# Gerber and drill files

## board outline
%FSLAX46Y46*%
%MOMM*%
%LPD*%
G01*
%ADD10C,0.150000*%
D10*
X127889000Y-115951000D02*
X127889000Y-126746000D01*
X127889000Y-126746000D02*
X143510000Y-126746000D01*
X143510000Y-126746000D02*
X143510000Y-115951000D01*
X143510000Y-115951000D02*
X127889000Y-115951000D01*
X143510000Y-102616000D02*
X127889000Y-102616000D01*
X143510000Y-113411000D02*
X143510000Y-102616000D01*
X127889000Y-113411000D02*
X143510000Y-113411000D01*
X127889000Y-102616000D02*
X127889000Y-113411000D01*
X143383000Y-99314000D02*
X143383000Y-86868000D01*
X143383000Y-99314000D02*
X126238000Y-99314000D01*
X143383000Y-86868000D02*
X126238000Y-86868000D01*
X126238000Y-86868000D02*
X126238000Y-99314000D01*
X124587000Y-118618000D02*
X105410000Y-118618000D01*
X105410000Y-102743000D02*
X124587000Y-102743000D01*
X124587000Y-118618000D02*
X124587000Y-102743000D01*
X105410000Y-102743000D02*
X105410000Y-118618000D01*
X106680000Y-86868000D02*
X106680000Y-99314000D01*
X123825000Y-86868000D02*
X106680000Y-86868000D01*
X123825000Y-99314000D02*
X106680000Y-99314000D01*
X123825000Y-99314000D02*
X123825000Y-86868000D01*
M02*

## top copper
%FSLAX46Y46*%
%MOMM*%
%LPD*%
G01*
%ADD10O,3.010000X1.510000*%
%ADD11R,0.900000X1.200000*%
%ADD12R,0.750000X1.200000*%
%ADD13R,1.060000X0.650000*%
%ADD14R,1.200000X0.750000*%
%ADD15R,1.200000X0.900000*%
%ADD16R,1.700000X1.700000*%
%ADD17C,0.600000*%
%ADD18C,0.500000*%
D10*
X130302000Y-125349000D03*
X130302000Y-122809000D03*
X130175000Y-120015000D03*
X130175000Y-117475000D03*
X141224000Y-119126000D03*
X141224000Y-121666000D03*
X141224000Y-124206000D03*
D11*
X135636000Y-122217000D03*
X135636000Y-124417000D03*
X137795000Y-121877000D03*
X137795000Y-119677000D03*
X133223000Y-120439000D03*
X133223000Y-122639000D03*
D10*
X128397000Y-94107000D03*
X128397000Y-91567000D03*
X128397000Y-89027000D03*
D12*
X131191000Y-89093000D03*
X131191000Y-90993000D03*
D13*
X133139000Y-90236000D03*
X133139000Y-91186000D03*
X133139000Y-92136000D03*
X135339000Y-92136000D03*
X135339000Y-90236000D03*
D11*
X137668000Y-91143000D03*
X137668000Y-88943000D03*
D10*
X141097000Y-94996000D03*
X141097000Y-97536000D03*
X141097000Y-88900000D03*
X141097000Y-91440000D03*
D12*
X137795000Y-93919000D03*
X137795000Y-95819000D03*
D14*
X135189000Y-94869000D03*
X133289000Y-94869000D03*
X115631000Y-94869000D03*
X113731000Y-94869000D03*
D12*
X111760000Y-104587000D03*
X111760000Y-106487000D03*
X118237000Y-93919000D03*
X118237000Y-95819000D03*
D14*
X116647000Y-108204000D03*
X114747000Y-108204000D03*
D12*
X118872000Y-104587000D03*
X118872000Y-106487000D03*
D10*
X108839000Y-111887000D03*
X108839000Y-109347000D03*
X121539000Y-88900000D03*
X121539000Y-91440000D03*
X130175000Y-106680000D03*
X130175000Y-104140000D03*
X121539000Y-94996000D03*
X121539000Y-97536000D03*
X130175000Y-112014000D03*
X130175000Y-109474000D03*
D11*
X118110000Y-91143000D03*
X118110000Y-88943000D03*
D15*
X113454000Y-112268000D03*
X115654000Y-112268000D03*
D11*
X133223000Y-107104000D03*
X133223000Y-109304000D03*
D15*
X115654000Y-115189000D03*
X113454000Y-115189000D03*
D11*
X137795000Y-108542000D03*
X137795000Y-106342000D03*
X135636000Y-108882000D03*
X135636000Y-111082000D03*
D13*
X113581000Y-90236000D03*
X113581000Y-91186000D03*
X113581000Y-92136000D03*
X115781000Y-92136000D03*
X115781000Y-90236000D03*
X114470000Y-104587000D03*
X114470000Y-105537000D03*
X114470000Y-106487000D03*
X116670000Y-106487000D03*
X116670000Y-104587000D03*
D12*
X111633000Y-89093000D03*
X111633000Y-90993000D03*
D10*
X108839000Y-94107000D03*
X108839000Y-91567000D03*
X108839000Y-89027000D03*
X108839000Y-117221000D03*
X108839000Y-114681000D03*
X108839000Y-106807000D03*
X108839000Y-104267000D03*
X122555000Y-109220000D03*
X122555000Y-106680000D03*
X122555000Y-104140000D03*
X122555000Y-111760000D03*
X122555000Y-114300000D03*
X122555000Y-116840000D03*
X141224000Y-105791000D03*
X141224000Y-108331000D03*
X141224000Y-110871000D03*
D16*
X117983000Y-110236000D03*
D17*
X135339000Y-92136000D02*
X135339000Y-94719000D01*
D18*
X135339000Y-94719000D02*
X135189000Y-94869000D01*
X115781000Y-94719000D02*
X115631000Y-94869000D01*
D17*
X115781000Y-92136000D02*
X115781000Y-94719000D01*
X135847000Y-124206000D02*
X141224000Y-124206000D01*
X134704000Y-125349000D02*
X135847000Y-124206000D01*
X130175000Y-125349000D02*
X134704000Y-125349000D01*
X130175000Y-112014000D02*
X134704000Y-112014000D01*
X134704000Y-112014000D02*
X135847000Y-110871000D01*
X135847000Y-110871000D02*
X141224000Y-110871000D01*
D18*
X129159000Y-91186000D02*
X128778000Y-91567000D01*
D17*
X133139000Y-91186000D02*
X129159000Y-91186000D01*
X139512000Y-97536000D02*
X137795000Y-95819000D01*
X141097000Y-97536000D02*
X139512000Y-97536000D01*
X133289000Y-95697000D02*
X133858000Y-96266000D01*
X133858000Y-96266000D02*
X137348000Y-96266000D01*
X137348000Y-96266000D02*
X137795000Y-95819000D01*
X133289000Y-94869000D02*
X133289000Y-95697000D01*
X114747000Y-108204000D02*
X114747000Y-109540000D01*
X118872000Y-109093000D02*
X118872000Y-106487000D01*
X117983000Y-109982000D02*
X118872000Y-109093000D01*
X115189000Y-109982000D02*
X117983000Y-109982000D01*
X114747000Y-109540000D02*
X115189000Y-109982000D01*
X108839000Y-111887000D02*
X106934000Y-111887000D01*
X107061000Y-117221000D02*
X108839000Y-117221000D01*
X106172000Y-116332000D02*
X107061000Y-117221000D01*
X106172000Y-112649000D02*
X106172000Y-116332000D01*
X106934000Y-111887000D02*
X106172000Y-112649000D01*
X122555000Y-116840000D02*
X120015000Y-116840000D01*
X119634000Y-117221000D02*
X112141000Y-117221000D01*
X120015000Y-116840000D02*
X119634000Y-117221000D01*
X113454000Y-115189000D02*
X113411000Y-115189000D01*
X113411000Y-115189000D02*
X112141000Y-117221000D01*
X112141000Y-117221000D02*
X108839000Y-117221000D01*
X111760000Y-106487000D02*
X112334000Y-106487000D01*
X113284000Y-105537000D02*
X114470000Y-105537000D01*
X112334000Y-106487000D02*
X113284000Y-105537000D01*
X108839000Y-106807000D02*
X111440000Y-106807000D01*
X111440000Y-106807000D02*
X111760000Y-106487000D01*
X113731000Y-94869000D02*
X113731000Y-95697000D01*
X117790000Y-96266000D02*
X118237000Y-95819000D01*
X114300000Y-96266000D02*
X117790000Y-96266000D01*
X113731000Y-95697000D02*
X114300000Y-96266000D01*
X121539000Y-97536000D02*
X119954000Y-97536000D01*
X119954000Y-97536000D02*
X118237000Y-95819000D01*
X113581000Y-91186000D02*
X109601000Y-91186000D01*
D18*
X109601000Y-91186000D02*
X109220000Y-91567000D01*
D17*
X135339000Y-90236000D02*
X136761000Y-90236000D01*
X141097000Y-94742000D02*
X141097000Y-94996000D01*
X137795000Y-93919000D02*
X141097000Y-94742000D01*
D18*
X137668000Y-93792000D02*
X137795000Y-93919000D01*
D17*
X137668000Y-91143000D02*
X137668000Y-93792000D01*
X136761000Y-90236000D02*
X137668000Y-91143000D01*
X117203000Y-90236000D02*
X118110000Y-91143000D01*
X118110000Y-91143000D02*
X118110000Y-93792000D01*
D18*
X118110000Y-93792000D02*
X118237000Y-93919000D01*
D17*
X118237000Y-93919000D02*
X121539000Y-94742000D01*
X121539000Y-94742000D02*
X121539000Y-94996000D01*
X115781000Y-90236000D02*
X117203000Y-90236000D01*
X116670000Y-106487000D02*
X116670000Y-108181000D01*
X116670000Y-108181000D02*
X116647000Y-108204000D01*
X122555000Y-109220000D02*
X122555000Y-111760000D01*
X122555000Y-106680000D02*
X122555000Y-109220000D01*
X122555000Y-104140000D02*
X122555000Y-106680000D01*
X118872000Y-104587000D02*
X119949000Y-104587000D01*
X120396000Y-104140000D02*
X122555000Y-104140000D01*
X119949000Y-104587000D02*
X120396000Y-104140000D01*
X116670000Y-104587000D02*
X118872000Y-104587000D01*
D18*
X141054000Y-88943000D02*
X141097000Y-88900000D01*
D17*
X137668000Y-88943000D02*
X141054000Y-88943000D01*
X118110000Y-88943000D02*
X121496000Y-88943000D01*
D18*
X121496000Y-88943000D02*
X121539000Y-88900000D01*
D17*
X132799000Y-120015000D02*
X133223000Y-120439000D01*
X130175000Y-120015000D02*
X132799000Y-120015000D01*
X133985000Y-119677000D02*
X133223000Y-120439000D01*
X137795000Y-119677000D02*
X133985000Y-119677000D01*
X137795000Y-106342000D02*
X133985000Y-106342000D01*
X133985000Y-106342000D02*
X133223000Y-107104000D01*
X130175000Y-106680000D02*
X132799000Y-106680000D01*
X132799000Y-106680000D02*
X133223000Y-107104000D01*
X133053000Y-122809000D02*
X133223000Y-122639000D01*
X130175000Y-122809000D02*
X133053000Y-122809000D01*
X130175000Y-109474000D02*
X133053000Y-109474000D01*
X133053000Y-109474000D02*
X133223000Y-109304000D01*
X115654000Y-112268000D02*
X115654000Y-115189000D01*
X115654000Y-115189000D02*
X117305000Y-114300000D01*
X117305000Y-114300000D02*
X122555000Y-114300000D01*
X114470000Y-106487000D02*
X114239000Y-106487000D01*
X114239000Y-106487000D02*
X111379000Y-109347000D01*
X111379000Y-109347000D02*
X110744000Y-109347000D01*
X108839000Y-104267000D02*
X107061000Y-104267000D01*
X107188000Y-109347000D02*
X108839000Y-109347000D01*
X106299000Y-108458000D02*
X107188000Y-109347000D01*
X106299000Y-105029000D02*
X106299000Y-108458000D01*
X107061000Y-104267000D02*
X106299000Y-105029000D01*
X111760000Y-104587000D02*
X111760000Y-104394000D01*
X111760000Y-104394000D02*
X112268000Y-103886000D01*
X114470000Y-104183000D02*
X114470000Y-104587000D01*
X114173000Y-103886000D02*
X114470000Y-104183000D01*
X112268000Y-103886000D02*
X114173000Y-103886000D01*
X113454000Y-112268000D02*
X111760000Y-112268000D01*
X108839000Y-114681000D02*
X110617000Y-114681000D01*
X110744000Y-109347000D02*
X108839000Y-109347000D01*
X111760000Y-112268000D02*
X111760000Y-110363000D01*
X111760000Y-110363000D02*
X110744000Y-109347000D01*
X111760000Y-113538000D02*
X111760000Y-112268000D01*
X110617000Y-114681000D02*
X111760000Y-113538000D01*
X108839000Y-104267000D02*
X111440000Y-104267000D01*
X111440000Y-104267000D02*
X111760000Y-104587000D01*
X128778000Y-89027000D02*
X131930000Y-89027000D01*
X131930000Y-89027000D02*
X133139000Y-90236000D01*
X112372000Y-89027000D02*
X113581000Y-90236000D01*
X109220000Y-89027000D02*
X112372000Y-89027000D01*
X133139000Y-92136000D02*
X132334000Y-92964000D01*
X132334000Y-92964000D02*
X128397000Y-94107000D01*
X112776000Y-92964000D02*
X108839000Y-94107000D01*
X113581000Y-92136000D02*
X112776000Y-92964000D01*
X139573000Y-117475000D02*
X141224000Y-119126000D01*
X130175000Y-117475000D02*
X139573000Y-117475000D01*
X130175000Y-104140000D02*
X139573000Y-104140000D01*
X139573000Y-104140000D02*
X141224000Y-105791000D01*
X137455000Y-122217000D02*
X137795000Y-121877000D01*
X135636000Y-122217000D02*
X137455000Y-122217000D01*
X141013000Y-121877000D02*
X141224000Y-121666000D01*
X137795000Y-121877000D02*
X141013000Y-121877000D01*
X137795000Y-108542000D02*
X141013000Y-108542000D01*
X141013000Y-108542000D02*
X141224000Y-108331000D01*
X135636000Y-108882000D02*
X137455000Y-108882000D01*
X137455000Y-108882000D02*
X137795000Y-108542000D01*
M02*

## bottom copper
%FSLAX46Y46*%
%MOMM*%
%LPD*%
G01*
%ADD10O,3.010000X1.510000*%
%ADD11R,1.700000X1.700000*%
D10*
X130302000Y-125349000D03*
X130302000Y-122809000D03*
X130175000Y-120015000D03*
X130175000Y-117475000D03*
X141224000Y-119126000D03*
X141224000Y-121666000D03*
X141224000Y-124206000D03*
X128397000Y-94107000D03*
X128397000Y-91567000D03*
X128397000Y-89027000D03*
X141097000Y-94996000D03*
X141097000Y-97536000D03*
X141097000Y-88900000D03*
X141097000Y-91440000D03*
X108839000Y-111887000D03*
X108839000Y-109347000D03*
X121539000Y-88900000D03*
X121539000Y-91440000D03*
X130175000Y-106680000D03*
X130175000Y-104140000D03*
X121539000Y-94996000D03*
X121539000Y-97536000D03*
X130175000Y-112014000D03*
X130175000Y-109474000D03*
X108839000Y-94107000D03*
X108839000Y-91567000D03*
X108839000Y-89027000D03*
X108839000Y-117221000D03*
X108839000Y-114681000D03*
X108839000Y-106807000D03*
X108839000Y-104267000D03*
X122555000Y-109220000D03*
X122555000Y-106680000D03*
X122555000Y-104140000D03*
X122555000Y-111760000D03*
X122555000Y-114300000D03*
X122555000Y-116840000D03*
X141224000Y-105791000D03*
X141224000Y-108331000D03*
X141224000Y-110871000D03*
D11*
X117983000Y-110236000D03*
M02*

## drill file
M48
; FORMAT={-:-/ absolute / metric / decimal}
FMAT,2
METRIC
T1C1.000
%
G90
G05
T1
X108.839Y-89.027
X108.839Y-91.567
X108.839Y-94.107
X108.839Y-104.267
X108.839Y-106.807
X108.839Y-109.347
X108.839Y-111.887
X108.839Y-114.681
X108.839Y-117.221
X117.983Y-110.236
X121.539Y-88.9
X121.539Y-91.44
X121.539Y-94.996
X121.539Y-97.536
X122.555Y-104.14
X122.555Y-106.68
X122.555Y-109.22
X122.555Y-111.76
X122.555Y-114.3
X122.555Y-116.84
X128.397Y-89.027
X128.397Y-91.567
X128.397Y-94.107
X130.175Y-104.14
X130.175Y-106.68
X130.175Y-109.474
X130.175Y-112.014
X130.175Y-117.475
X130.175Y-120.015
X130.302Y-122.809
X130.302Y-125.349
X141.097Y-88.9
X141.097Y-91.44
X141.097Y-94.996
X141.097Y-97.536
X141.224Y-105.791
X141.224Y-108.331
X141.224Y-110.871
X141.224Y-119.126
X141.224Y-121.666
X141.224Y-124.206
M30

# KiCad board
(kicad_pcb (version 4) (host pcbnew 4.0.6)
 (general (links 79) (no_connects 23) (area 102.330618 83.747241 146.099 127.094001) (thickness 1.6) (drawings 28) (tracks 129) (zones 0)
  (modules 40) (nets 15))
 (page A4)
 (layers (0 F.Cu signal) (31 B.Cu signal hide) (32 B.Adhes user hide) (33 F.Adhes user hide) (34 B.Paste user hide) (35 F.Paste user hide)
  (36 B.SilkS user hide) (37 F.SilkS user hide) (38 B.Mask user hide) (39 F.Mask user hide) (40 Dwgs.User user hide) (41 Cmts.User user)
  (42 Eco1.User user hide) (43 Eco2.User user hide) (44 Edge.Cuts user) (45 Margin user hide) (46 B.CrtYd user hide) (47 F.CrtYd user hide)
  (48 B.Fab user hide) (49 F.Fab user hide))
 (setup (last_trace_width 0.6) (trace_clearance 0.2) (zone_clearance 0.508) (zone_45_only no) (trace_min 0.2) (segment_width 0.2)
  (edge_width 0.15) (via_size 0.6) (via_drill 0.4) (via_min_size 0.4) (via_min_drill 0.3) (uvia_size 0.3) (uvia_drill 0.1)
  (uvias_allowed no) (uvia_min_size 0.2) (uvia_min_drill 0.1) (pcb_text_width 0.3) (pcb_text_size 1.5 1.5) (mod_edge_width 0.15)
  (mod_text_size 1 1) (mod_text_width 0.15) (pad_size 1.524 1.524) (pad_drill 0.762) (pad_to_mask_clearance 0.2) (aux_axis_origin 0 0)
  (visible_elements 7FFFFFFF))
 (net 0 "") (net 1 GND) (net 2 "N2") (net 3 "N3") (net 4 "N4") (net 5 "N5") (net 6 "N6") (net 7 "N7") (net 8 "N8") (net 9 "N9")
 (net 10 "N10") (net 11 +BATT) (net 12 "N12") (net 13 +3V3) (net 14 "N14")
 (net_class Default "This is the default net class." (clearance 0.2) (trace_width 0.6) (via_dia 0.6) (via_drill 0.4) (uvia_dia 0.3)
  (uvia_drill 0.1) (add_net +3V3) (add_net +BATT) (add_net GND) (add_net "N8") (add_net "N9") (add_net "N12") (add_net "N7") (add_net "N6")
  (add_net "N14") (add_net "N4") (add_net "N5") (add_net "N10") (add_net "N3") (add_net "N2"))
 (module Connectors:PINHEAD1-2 (layer F.Cu) (at 130.302 125.349 90)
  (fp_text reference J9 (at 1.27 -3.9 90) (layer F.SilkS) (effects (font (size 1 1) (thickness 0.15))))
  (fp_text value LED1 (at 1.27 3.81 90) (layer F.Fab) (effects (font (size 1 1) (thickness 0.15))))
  (pad 1 thru_hole oval (at 0 0 90) (size 1.51 3.01) (drill 1) (layers *.Cu *.Mask) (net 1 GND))
  (pad 2 thru_hole oval (at 2.54 0 90) (size 1.51 3.01) (drill 1) (layers *.Cu *.Mask) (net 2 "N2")))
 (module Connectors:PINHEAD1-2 (layer F.Cu) (at 130.175 120.015 90)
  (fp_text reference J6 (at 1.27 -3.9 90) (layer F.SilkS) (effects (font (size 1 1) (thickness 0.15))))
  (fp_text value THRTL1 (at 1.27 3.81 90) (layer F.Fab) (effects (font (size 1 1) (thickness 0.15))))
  (pad 1 thru_hole oval (at 0 0 90) (size 1.51 3.01) (drill 1) (layers *.Cu *.Mask) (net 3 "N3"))
  (pad 2 thru_hole oval (at 2.54 0 90) (size 1.51 3.01) (drill 1) (layers *.Cu *.Mask) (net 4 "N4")))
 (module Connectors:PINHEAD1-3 (layer F.Cu) (at 141.224 119.126 270)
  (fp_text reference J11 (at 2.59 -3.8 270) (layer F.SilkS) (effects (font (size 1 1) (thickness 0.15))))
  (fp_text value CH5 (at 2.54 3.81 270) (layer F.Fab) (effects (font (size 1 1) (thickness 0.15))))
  (pad 1 thru_hole oval (at 0 0 270) (size 1.51 3.01) (drill 1) (layers *.Cu *.Mask) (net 4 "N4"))
  (pad 2 thru_hole oval (at 2.54 0 270) (size 1.51 3.01) (drill 1) (layers *.Cu *.Mask) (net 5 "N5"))
  (pad 3 thru_hole oval (at 5.08 0 270) (size 1.51 3.01) (drill 1) (layers *.Cu *.Mask) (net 1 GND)))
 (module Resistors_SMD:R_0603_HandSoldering (layer F.Cu) (at 135.636 123.317 270)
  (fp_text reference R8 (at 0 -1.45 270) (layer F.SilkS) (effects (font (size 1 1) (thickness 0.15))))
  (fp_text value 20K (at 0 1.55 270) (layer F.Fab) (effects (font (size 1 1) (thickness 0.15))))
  (pad 1 smd rect (at -1.1 0 270) (size 1.2 0.9) (layers F.Cu F.Paste F.Mask) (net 5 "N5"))
  (pad 2 smd rect (at 1.1 0 270) (size 1.2 0.9) (layers F.Cu F.Paste F.Mask) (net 1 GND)))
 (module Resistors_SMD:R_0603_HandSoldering (layer F.Cu) (at 137.795 120.777 90)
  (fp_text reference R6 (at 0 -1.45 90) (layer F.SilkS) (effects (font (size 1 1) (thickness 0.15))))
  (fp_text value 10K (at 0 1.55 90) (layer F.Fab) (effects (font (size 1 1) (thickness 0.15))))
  (pad 1 smd rect (at -1.1 0 90) (size 1.2 0.9) (layers F.Cu F.Paste F.Mask) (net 5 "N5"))
  (pad 2 smd rect (at 1.1 0 90) (size 1.2 0.9) (layers F.Cu F.Paste F.Mask) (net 3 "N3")))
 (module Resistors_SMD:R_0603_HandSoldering (layer F.Cu) (at 133.223 121.539 270)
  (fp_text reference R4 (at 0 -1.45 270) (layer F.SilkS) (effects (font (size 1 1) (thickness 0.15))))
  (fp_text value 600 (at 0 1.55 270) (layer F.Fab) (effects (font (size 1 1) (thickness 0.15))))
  (pad 1 smd rect (at -1.1 0 270) (size 1.2 0.9) (layers F.Cu F.Paste F.Mask) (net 3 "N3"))
  (pad 2 smd rect (at 1.1 0 270) (size 1.2 0.9) (layers F.Cu F.Paste F.Mask) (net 2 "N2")))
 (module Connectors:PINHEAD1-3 (layer F.Cu) (at 128.397 94.107 90)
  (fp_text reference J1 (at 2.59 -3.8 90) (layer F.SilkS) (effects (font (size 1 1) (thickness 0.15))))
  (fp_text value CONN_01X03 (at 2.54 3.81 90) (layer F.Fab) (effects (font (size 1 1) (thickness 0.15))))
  (pad 1 thru_hole oval (at 0 0 90) (size 1.51 3.01) (drill 1) (layers *.Cu *.Mask) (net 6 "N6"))
  (pad 2 thru_hole oval (at 2.54 0 90) (size 1.51 3.01) (drill 1) (layers *.Cu *.Mask) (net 1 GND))
  (pad 3 thru_hole oval (at 5.08 0 90) (size 1.51 3.01) (drill 1) (layers *.Cu *.Mask) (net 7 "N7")))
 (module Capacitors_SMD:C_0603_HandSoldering (layer F.Cu) (at 131.191 90.043 270)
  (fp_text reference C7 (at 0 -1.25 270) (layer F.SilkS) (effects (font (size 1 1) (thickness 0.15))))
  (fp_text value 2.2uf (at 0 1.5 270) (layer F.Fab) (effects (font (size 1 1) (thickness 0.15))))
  (pad 1 smd rect (at -0.95 0 270) (size 1.2 0.75) (layers F.Cu F.Paste F.Mask) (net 7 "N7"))
  (pad 2 smd rect (at 0.95 0 270) (size 1.2 0.75) (layers F.Cu F.Paste F.Mask) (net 1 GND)))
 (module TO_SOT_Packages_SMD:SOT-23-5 (layer F.Cu) (at 134.239 91.186)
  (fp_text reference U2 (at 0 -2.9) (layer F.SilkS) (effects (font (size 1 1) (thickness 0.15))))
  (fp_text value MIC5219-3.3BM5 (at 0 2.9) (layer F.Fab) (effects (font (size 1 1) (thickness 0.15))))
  (pad 1 smd rect (at -1.1 -0.95) (size 1.06 0.65) (layers F.Cu F.Paste F.Mask) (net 7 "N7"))
  (pad 2 smd rect (at -1.1 0) (size 1.06 0.65) (layers F.Cu F.Paste F.Mask) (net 1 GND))
  (pad 3 smd rect (at -1.1 0.95) (size 1.06 0.65) (layers F.Cu F.Paste F.Mask) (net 6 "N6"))
  (pad 4 smd rect (at 1.1 0.95) (size 1.06 0.65) (layers F.Cu F.Paste F.Mask) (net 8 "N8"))
  (pad 5 smd rect (at 1.1 -0.95) (size 1.06 0.65) (layers F.Cu F.Paste F.Mask) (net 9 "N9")))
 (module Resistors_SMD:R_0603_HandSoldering (layer F.Cu) (at 137.668 90.043 90)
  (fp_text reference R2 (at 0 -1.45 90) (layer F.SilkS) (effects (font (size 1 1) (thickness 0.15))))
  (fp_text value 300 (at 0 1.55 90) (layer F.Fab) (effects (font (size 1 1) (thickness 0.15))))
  (pad 1 smd rect (at -1.1 0 90) (size 1.2 0.9) (layers F.Cu F.Paste F.Mask) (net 9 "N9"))
  (pad 2 smd rect (at 1.1 0 90) (size 1.2 0.9) (layers F.Cu F.Paste F.Mask) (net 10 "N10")))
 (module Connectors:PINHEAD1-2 (layer F.Cu) (at 141.097 94.996 270)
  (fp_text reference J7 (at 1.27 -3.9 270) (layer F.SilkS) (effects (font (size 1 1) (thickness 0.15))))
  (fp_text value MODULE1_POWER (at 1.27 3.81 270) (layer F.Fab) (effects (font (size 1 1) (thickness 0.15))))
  (pad 1 thru_hole oval (at 0 0 270) (size 1.51 3.01) (drill 1) (layers *.Cu *.Mask) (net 9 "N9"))
  (pad 2 thru_hole oval (at 2.54 0 270) (size 1.51 3.01) (drill 1) (layers *.Cu *.Mask) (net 1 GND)))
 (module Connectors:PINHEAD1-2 (layer F.Cu) (at 141.097 88.9 270)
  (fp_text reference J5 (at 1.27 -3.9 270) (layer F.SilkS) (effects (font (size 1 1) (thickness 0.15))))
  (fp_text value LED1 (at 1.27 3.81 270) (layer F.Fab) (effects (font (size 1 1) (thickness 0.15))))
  (pad 1 thru_hole oval (at 0 0 270) (size 1.51 3.01) (drill 1) (layers *.Cu *.Mask) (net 10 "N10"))
  (pad 2 thru_hole oval (at 2.54 0 270) (size 1.51 3.01) (drill 1) (layers *.Cu *.Mask) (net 1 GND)))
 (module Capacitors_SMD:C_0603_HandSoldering (layer F.Cu) (at 137.795 94.869 270)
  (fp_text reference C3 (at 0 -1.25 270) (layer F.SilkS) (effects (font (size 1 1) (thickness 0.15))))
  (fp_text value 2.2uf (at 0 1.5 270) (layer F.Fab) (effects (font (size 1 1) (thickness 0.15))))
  (pad 1 smd rect (at -0.95 0 270) (size 1.2 0.75) (layers F.Cu F.Paste F.Mask) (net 9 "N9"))
  (pad 2 smd rect (at 0.95 0 270) (size 1.2 0.75) (layers F.Cu F.Paste F.Mask) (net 1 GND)))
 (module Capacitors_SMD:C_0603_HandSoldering (layer F.Cu) (at 134.239 94.869 180)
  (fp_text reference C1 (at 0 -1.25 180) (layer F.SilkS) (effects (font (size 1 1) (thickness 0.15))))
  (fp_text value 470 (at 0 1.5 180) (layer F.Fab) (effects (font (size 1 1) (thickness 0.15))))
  (pad 1 smd rect (at -0.95 0 180) (size 1.2 0.75) (layers F.Cu F.Paste F.Mask) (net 8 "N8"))
  (pad 2 smd rect (at 0.95 0 180) (size 1.2 0.75) (layers F.Cu F.Paste F.Mask) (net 1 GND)))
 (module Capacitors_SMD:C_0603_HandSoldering (layer F.Cu) (at 114.681 94.869 180)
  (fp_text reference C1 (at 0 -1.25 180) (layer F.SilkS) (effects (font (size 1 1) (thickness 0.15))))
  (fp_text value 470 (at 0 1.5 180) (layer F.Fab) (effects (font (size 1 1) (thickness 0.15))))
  (pad 1 smd rect (at -0.95 0 180) (size 1.2 0.75) (layers F.Cu F.Paste F.Mask) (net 8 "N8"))
  (pad 2 smd rect (at 0.95 0 180) (size 1.2 0.75) (layers F.Cu F.Paste F.Mask) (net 1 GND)))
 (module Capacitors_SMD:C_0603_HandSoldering (layer F.Cu) (at 111.76 105.537 270)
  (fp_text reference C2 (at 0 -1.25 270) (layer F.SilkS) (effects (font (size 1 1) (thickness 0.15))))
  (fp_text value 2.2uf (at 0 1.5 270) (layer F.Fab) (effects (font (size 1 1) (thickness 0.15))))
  (pad 1 smd rect (at -0.95 0 270) (size 1.2 0.75) (layers F.Cu F.Paste F.Mask) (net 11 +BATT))
  (pad 2 smd rect (at 0.95 0 270) (size 1.2 0.75) (layers F.Cu F.Paste F.Mask) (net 1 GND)))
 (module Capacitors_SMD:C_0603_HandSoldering (layer F.Cu) (at 118.237 94.869 270)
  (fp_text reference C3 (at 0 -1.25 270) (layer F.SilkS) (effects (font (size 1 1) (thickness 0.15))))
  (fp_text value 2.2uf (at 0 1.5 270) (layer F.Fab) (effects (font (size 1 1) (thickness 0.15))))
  (pad 1 smd rect (at -0.95 0 270) (size 1.2 0.75) (layers F.Cu F.Paste F.Mask) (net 9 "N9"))
  (pad 2 smd rect (at 0.95 0 270) (size 1.2 0.75) (layers F.Cu F.Paste F.Mask) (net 1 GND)))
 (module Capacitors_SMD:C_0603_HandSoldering (layer F.Cu) (at 115.697 108.204 180)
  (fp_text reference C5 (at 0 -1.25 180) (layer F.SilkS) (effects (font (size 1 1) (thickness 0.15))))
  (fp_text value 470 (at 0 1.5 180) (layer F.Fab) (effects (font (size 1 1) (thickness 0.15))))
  (pad 1 smd rect (at -0.95 0 180) (size 1.2 0.75) (layers F.Cu F.Paste F.Mask) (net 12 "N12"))
  (pad 2 smd rect (at 0.95 0 180) (size 1.2 0.75) (layers F.Cu F.Paste F.Mask) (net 1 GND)))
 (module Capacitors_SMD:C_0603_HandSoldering (layer F.Cu) (at 118.872 105.537 270)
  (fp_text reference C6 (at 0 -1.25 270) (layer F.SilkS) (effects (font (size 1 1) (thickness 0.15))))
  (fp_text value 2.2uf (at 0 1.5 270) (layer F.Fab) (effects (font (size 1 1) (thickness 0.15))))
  (pad 1 smd rect (at -0.95 0 270) (size 1.2 0.75) (layers F.Cu F.Paste F.Mask) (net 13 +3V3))
  (pad 2 smd rect (at 0.95 0 270) (size 1.2 0.75) (layers F.Cu F.Paste F.Mask) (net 1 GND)))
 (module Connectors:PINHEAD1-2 (layer F.Cu) (at 108.839 111.887 90)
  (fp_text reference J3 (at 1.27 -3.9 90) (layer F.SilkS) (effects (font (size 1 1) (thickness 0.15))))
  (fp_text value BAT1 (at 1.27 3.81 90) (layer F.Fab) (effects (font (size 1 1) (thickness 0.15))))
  (pad 1 thru_hole oval (at 0 0 90) (size 1.51 3.01) (drill 1) (layers *.Cu *.Mask) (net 1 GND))
  (pad 2 thru_hole oval (at 2.54 0 90) (size 1.51 3.01) (drill 1) (layers *.Cu *.Mask) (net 11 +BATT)))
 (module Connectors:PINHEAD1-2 (layer F.Cu) (at 121.539 88.9 270)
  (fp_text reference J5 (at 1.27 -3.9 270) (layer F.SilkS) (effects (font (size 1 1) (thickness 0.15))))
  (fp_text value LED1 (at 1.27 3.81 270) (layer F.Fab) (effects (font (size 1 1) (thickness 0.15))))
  (pad 1 thru_hole oval (at 0 0 270) (size 1.51 3.01) (drill 1) (layers *.Cu *.Mask) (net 10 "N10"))
  (pad 2 thru_hole oval (at 2.54 0 270) (size 1.51 3.01) (drill 1) (layers *.Cu *.Mask) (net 1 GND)))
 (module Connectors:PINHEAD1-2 (layer F.Cu) (at 130.175 106.68 90)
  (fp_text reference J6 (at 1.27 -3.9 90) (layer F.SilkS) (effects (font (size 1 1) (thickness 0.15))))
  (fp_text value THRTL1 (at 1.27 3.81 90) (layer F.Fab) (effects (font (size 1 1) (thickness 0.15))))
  (pad 1 thru_hole oval (at 0 0 90) (size 1.51 3.01) (drill 1) (layers *.Cu *.Mask) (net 3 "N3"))
  (pad 2 thru_hole oval (at 2.54 0 90) (size 1.51 3.01) (drill 1) (layers *.Cu *.Mask) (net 4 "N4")))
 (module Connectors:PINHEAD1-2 (layer F.Cu) (at 121.539 94.996 270)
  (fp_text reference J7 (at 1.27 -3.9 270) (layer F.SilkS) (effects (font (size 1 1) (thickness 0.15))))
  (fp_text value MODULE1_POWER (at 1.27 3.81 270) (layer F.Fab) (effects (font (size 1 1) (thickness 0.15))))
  (pad 1 thru_hole oval (at 0 0 270) (size 1.51 3.01) (drill 1) (layers *.Cu *.Mask) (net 9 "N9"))
  (pad 2 thru_hole oval (at 2.54 0 270) (size 1.51 3.01) (drill 1) (layers *.Cu *.Mask) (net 1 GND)))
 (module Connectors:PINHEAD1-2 (layer F.Cu) (at 130.175 112.014 90)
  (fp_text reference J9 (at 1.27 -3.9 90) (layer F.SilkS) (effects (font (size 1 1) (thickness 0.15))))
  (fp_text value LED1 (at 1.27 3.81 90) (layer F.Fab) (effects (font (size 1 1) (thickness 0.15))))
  (pad 1 thru_hole oval (at 0 0 90) (size 1.51 3.01) (drill 1) (layers *.Cu *.Mask) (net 1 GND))
  (pad 2 thru_hole oval (at 2.54 0 90) (size 1.51 3.01) (drill 1) (layers *.Cu *.Mask) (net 2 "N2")))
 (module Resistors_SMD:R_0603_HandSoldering (layer F.Cu) (at 118.11 90.043 90)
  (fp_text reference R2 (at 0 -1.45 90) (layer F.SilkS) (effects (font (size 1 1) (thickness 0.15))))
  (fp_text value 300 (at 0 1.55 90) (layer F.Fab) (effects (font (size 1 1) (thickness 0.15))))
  (pad 1 smd rect (at -1.1 0 90) (size 1.2 0.9) (layers F.Cu F.Paste F.Mask) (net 9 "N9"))
  (pad 2 smd rect (at 1.1 0 90) (size 1.2 0.9) (layers F.Cu F.Paste F.Mask) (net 10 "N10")))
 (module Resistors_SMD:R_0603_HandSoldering (layer F.Cu) (at 114.554 112.268)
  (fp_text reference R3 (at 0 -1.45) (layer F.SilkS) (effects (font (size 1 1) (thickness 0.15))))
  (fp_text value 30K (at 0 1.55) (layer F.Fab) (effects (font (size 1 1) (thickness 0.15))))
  (pad 1 smd rect (at -1.1 0) (size 1.2 0.9) (layers F.Cu F.Paste F.Mask) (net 11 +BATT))
  (pad 2 smd rect (at 1.1 0) (size 1.2 0.9) (layers F.Cu F.Paste F.Mask) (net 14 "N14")))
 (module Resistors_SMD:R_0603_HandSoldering (layer F.Cu) (at 133.223 108.204 270)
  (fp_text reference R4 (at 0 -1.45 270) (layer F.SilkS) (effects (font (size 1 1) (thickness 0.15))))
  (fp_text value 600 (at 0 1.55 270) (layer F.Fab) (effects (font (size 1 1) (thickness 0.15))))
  (pad 1 smd rect (at -1.1 0 270) (size 1.2 0.9) (layers F.Cu F.Paste F.Mask) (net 3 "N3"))
  (pad 2 smd rect (at 1.1 0 270) (size 1.2 0.9) (layers F.Cu F.Paste F.Mask) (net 2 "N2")))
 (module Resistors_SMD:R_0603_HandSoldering (layer F.Cu) (at 114.554 115.189 180)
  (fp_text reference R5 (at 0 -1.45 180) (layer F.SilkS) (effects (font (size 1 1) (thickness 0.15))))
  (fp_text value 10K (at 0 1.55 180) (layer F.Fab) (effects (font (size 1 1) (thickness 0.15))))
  (pad 1 smd rect (at -1.1 0 180) (size 1.2 0.9) (layers F.Cu F.Paste F.Mask) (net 14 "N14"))
  (pad 2 smd rect (at 1.1 0 180) (size 1.2 0.9) (layers F.Cu F.Paste F.Mask) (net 1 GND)))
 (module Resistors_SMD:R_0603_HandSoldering (layer F.Cu) (at 137.795 107.442 90)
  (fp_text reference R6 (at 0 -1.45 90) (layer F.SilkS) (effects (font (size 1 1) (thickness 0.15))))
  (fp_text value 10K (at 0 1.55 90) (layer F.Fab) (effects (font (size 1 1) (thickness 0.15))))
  (pad 1 smd rect (at -1.1 0 90) (size 1.2 0.9) (layers F.Cu F.Paste F.Mask) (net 5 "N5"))
  (pad 2 smd rect (at 1.1 0 90) (size 1.2 0.9) (layers F.Cu F.Paste F.Mask) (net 3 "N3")))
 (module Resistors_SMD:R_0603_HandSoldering (layer F.Cu) (at 135.636 109.982 270)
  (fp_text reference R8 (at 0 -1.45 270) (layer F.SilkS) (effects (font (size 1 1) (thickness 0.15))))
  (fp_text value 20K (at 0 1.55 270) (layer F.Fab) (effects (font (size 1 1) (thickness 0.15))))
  (pad 1 smd rect (at -1.1 0 270) (size 1.2 0.9) (layers F.Cu F.Paste F.Mask) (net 5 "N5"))
  (pad 2 smd rect (at 1.1 0 270) (size 1.2 0.9) (layers F.Cu F.Paste F.Mask) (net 1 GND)))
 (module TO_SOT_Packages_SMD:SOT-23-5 (layer F.Cu) (at 114.681 91.186)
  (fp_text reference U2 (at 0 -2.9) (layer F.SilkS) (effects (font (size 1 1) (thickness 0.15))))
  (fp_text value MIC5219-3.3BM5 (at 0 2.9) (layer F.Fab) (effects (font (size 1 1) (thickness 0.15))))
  (pad 1 smd rect (at -1.1 -0.95) (size 1.06 0.65) (layers F.Cu F.Paste F.Mask) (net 7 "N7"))
  (pad 2 smd rect (at -1.1 0) (size 1.06 0.65) (layers F.Cu F.Paste F.Mask) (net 1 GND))
  (pad 3 smd rect (at -1.1 0.95) (size 1.06 0.65) (layers F.Cu F.Paste F.Mask) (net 6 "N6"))
  (pad 4 smd rect (at 1.1 0.95) (size 1.06 0.65) (layers F.Cu F.Paste F.Mask) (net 8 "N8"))
  (pad 5 smd rect (at 1.1 -0.95) (size 1.06 0.65) (layers F.Cu F.Paste F.Mask) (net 9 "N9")))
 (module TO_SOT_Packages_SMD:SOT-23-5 (layer F.Cu) (at 115.57 105.537)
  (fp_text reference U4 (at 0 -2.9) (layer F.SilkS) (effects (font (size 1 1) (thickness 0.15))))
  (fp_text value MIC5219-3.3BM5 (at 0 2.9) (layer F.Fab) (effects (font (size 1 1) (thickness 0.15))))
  (pad 1 smd rect (at -1.1 -0.95) (size 1.06 0.65) (layers F.Cu F.Paste F.Mask) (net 11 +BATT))
  (pad 2 smd rect (at -1.1 0) (size 1.06 0.65) (layers F.Cu F.Paste F.Mask) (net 1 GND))
  (pad 3 smd rect (at -1.1 0.95) (size 1.06 0.65) (layers F.Cu F.Paste F.Mask) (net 11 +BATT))
  (pad 4 smd rect (at 1.1 0.95) (size 1.06 0.65) (layers F.Cu F.Paste F.Mask) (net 12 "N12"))
  (pad 5 smd rect (at 1.1 -0.95) (size 1.06 0.65) (layers F.Cu F.Paste F.Mask) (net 13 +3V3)))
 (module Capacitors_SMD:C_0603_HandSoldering (layer F.Cu) (at 111.633 90.043 270)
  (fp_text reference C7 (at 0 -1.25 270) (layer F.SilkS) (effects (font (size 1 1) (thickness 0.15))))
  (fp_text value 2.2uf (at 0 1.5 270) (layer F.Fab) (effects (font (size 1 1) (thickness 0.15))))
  (pad 1 smd rect (at -0.95 0 270) (size 1.2 0.75) (layers F.Cu F.Paste F.Mask) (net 7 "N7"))
  (pad 2 smd rect (at 0.95 0 270) (size 1.2 0.75) (layers F.Cu F.Paste F.Mask) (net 1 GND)))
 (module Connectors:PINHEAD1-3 (layer F.Cu) (at 108.839 94.107 90)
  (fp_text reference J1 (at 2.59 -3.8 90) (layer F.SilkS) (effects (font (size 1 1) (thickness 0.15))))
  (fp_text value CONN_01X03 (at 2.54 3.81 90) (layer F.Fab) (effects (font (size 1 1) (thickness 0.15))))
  (pad 1 thru_hole oval (at 0 0 90) (size 1.51 3.01) (drill 1) (layers *.Cu *.Mask) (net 6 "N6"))
  (pad 2 thru_hole oval (at 2.54 0 90) (size 1.51 3.01) (drill 1) (layers *.Cu *.Mask) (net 1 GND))
  (pad 3 thru_hole oval (at 5.08 0 90) (size 1.51 3.01) (drill 1) (layers *.Cu *.Mask) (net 7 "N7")))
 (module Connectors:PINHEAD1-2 (layer F.Cu) (at 108.839 117.221 90)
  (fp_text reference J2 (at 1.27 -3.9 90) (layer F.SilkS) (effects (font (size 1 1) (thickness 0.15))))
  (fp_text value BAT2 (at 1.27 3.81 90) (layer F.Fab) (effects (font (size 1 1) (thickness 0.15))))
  (pad 1 thru_hole oval (at 0 0 90) (size 1.51 3.01) (drill 1) (layers *.Cu *.Mask) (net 1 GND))
  (pad 2 thru_hole oval (at 2.54 0 90) (size 1.51 3.01) (drill 1) (layers *.Cu *.Mask) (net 11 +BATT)))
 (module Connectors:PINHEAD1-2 (layer F.Cu) (at 108.839 106.807 90)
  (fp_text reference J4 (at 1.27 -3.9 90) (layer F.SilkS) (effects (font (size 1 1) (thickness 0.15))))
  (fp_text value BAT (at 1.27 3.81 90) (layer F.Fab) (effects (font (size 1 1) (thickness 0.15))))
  (pad 1 thru_hole oval (at 0 0 90) (size 1.51 3.01) (drill 1) (layers *.Cu *.Mask) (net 1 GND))
  (pad 2 thru_hole oval (at 2.54 0 90) (size 1.51 3.01) (drill 1) (layers *.Cu *.Mask) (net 11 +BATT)))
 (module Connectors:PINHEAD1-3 (layer F.Cu) (at 122.555 109.22 90)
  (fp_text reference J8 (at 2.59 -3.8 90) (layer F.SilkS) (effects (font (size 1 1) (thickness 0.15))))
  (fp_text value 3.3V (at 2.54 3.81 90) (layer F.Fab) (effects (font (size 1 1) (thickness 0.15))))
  (pad 1 thru_hole oval (at 0 0 90) (size 1.51 3.01) (drill 1) (layers *.Cu *.Mask) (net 13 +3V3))
  (pad 2 thru_hole oval (at 2.54 0 90) (size 1.51 3.01) (drill 1) (layers *.Cu *.Mask) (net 13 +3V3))
  (pad 3 thru_hole oval (at 5.08 0 90) (size 1.51 3.01) (drill 1) (layers *.Cu *.Mask) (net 13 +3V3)))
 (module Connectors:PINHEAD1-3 (layer F.Cu) (at 122.555 111.76 270)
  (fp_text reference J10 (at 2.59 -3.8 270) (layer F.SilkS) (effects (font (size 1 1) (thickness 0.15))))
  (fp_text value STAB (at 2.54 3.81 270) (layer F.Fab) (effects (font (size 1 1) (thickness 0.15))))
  (pad 1 thru_hole oval (at 0 0 270) (size 1.51 3.01) (drill 1) (layers *.Cu *.Mask) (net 13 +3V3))
  (pad 2 thru_hole oval (at 2.54 0 270) (size 1.51 3.01) (drill 1) (layers *.Cu *.Mask) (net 14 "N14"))
  (pad 3 thru_hole oval (at 5.08 0 270) (size 1.51 3.01) (drill 1) (layers *.Cu *.Mask) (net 1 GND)))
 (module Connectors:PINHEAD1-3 (layer F.Cu) (at 141.224 105.791 270)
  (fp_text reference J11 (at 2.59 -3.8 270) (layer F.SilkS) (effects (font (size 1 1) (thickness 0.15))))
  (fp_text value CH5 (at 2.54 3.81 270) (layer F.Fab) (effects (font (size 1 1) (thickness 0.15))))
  (pad 1 thru_hole oval (at 0 0 270) (size 1.51 3.01) (drill 1) (layers *.Cu *.Mask) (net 4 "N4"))
  (pad 2 thru_hole oval (at 2.54 0 270) (size 1.51 3.01) (drill 1) (layers *.Cu *.Mask) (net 5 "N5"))
  (pad 3 thru_hole oval (at 5.08 0 270) (size 1.51 3.01) (drill 1) (layers *.Cu *.Mask) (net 1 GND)))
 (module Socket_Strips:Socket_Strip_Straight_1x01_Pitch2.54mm (layer F.Cu) (at 117.983 110.236)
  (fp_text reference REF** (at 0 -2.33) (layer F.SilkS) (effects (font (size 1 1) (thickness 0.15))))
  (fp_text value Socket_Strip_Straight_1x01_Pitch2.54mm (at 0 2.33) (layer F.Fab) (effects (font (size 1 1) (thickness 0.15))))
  (pad 1 thru_hole rect (at 0 0) (size 1.7 1.7) (drill 1) (layers *.Cu *.Mask)))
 (gr_line (start 127.889 115.951) (end 127.889 126.746) (angle 90) (layer Edge.Cuts) (width 0.15))
 (gr_line (start 127.889 126.746) (end 143.51 126.746) (angle 90) (layer Edge.Cuts) (width 0.15))
 (gr_line (start 143.51 126.746) (end 143.51 115.951) (angle 90) (layer Edge.Cuts) (width 0.15))
 (gr_line (start 143.51 115.951) (end 127.889 115.951) (angle 90) (layer Edge.Cuts) (width 0.15))
 (gr_line (start 143.51 102.616) (end 127.889 102.616) (angle 90) (layer Edge.Cuts) (width 0.15))
 (gr_line (start 143.51 113.411) (end 143.51 102.616) (angle 90) (layer Edge.Cuts) (width 0.15))
 (gr_line (start 127.889 113.411) (end 143.51 113.411) (angle 90) (layer Edge.Cuts) (width 0.15))
 (gr_line (start 127.889 102.616) (end 127.889 113.411) (angle 90) (layer Edge.Cuts) (width 0.15))
 (gr_line (start 143.383 99.314) (end 143.383 86.868) (angle 90) (layer Edge.Cuts) (width 0.15))
 (gr_line (start 143.383 99.314) (end 126.238 99.314) (angle 90) (layer Edge.Cuts) (width 0.15))
 (gr_line (start 143.383 86.868) (end 126.238 86.868) (angle 90) (layer Edge.Cuts) (width 0.15))
 (gr_line (start 126.238 86.868) (end 126.238 99.314) (angle 90) (layer Edge.Cuts) (width 0.15))
 (gr_line (start 124.587 118.618) (end 105.41 118.618) (angle 90) (layer Edge.Cuts) (width 0.15))
 (gr_line (start 105.41 102.743) (end 124.587 102.743) (angle 90) (layer Edge.Cuts) (width 0.15))
 (gr_line (start 124.587 118.618) (end 124.587 102.743) (angle 90) (layer Edge.Cuts) (width 0.15))
 (gr_line (start 105.41 102.743) (end 105.41 118.618) (angle 90) (layer Edge.Cuts) (width 0.15))
 (gr_line (start 106.68 86.868) (end 106.68 99.314) (angle 90) (layer Edge.Cuts) (width 0.15))
 (gr_line (start 123.825 86.868) (end 106.68 86.868) (angle 90) (layer Edge.Cuts) (width 0.15))
 (gr_line (start 123.825 99.314) (end 106.68 99.314) (angle 90) (layer Edge.Cuts) (width 0.15))
 (gr_line (start 123.825 99.314) (end 123.825 86.868) (angle 90) (layer Edge.Cuts) (width 0.15))
 (segment (start 135.339 92.136) (end 135.339 94.719) (width 0.6) (layer F.Cu) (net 8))
 (segment (start 135.339 94.719) (end 135.189 94.869) (width 0.5) (layer F.Cu) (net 8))
 (segment (start 115.781 94.719) (end 115.631 94.869) (width 0.5) (layer F.Cu) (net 8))
 (segment (start 115.781 92.136) (end 115.781 94.719) (width 0.6) (layer F.Cu) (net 8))
 (segment (start 135.847 124.206) (end 141.224 124.206) (width 0.6) (layer F.Cu) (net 1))
 (segment (start 134.704 125.349) (end 135.847 124.206) (width 0.6) (layer F.Cu) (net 1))
 (segment (start 130.175 125.349) (end 134.704 125.349) (width 0.6) (layer F.Cu) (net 1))
 (segment (start 130.175 112.014) (end 134.704 112.014) (width 0.6) (layer F.Cu) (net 1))
 (segment (start 134.704 112.014) (end 135.847 110.871) (width 0.6) (layer F.Cu) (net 1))
 (segment (start 135.847 110.871) (end 141.224 110.871) (width 0.6) (layer F.Cu) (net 1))
 (segment (start 129.159 91.186) (end 128.778 91.567) (width 0.5) (layer F.Cu) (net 1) (status 30))
 (segment (start 133.139 91.186) (end 129.159 91.186) (width 0.6) (layer F.Cu) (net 1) (status 20))
 (segment (start 139.512 97.536) (end 137.795 95.819) (width 0.6) (layer F.Cu) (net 1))
 (segment (start 141.097 97.536) (end 139.512 97.536) (width 0.6) (layer F.Cu) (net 1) (status 10))
 (segment (start 133.289 95.697) (end 133.858 96.266) (width 0.6) (layer F.Cu) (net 1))
 (segment (start 133.858 96.266) (end 137.348 96.266) (width 0.6) (layer F.Cu) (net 1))
 (segment (start 137.348 96.266) (end 137.795 95.819) (width 0.6) (layer F.Cu) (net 1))
 (segment (start 133.289 94.869) (end 133.289 95.697) (width 0.6) (layer F.Cu) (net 1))
 (segment (start 114.747 108.204) (end 114.747 109.54) (width 0.6) (layer F.Cu) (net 1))
 (segment (start 118.872 109.093) (end 118.872 106.487) (width 0.6) (layer F.Cu) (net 1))
 (segment (start 117.983 109.982) (end 118.872 109.093) (width 0.6) (layer F.Cu) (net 1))
 (segment (start 115.189 109.982) (end 117.983 109.982) (width 0.6) (layer F.Cu) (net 1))
 (segment (start 114.747 109.54) (end 115.189 109.982) (width 0.6) (layer F.Cu) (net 1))
 (segment (start 108.839 111.887) (end 106.934 111.887) (width 0.6) (layer F.Cu) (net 1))
 (segment (start 107.061 117.221) (end 108.839 117.221) (width 0.6) (layer F.Cu) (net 1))
 (segment (start 106.172 116.332) (end 107.061 117.221) (width 0.6) (layer F.Cu) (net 1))
 (segment (start 106.172 112.649) (end 106.172 116.332) (width 0.6) (layer F.Cu) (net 1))
 (segment (start 106.934 111.887) (end 106.172 112.649) (width 0.6) (layer F.Cu) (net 1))
 (segment (start 122.555 116.84) (end 120.015 116.84) (width 0.6) (layer F.Cu) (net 1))
 (segment (start 119.634 117.221) (end 112.141 117.221) (width 0.6) (layer F.Cu) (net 1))
 (segment (start 120.015 116.84) (end 119.634 117.221) (width 0.6) (layer F.Cu) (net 1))
 (segment (start 113.454 115.189) (end 113.411 115.189) (width 0.6) (layer F.Cu) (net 1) (status 30))
 (segment (start 113.411 115.189) (end 112.141 117.221) (width 0.6) (layer F.Cu) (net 1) (status 10))
 (segment (start 112.141 117.221) (end 108.839 117.221) (width 0.6) (layer F.Cu) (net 1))
 (segment (start 111.76 106.487) (end 112.334 106.487) (width 0.6) (layer F.Cu) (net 1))
 (segment (start 113.284 105.537) (end 114.47 105.537) (width 0.6) (layer F.Cu) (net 1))
 (segment (start 112.334 106.487) (end 113.284 105.537) (width 0.6) (layer F.Cu) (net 1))
 (segment (start 108.839 106.807) (end 111.44 106.807) (width 0.6) (layer F.Cu) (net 1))
 (segment (start 111.44 106.807) (end 111.76 106.487) (width 0.6) (layer F.Cu) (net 1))
 (segment (start 113.731 94.869) (end 113.731 95.697) (width 0.6) (layer F.Cu) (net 1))
 (segment (start 117.79 96.266) (end 118.237 95.819) (width 0.6) (layer F.Cu) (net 1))
 (segment (start 114.3 96.266) (end 117.79 96.266) (width 0.6) (layer F.Cu) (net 1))
 (segment (start 113.731 95.697) (end 114.3 96.266) (width 0.6) (layer F.Cu) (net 1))
 (segment (start 121.539 97.536) (end 119.954 97.536) (width 0.6) (layer F.Cu) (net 1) (status 10))
 (segment (start 119.954 97.536) (end 118.237 95.819) (width 0.6) (layer F.Cu) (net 1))
 (segment (start 113.581 91.186) (end 109.601 91.186) (width 0.6) (layer F.Cu) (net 1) (status 20))
 (segment (start 109.601 91.186) (end 109.22 91.567) (width 0.5) (layer F.Cu) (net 1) (status 30))
 (segment (start 135.339 90.236) (end 136.761 90.236) (width 0.6) (layer F.Cu) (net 9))
 (segment (start 141.097 94.742) (end 141.097 94.996) (width 0.6) (layer F.Cu) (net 9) (status 20))
 (segment (start 137.795 93.919) (end 141.097 94.742) (width 0.6) (layer F.Cu) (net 9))
 (segment (start 137.668 93.792) (end 137.795 93.919) (width 0.5) (layer F.Cu) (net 9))
 (segment (start 137.668 91.143) (end 137.668 93.792) (width 0.6) (layer F.Cu) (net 9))
 (segment (start 136.761 90.236) (end 137.668 91.143) (width 0.6) (layer F.Cu) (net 9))
 (segment (start 117.203 90.236) (end 118.11 91.143) (width 0.6) (layer F.Cu) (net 9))
 (segment (start 118.11 91.143) (end 118.11 93.792) (width 0.6) (layer F.Cu) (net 9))
 (segment (start 118.11 93.792) (end 118.237 93.919) (width 0.5) (layer F.Cu) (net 9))
 (segment (start 118.237 93.919) (end 121.539 94.742) (width 0.6) (layer F.Cu) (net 9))
 (segment (start 121.539 94.742) (end 121.539 94.996) (width 0.6) (layer F.Cu) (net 9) (status 20))
 (segment (start 115.781 90.236) (end 117.203 90.236) (width 0.6) (layer F.Cu) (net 9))
 (segment (start 116.67 106.487) (end 116.67 108.181) (width 0.6) (layer F.Cu) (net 12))
 (segment (start 116.67 108.181) (end 116.647 108.204) (width 0.6) (layer F.Cu) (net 12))
 (segment (start 122.555 109.22) (end 122.555 111.76) (width 0.6) (layer F.Cu) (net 13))
 (segment (start 122.555 106.68) (end 122.555 109.22) (width 0.6) (layer F.Cu) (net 13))
 (segment (start 122.555 104.14) (end 122.555 106.68) (width 0.6) (layer F.Cu) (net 13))
 (segment (start 118.872 104.587) (end 119.949 104.587) (width 0.6) (layer F.Cu) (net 13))
 (segment (start 120.396 104.14) (end 122.555 104.14) (width 0.6) (layer F.Cu) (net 13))
 (segment (start 119.949 104.587) (end 120.396 104.14) (width 0.6) (layer F.Cu) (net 13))
 (segment (start 116.67 104.587) (end 118.872 104.587) (width 0.6) (layer F.Cu) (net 13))
 (segment (start 141.054 88.943) (end 141.097 88.9) (width 0.5) (layer F.Cu) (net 10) (status 30))
 (segment (start 137.668 88.943) (end 141.054 88.943) (width 0.6) (layer F.Cu) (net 10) (status 20))
 (segment (start 118.11 88.943) (end 121.496 88.943) (width 0.6) (layer F.Cu) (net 10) (status 20))
 (segment (start 121.496 88.943) (end 121.539 88.9) (width 0.5) (layer F.Cu) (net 10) (status 30))
 (segment (start 132.799 120.015) (end 133.223 120.439) (width 0.6) (layer F.Cu) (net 3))
 (segment (start 130.175 120.015) (end 132.799 120.015) (width 0.6) (layer F.Cu) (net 3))
 (segment (start 133.985 119.677) (end 133.223 120.439) (width 0.6) (layer F.Cu) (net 3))
 (segment (start 137.795 119.677) (end 133.985 119.677) (width 0.6) (layer F.Cu) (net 3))
 (segment (start 137.795 106.342) (end 133.985 106.342) (width 0.6) (layer F.Cu) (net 3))
 (segment (start 133.985 106.342) (end 133.223 107.104) (width 0.6) (layer F.Cu) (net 3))
 (segment (start 130.175 106.68) (end 132.799 106.68) (width 0.6) (layer F.Cu) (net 3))
 (segment (start 132.799 106.68) (end 133.223 107.104) (width 0.6) (layer F.Cu) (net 3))
 (segment (start 133.053 122.809) (end 133.223 122.639) (width 0.6) (layer F.Cu) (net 2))
 (segment (start 130.175 122.809) (end 133.053 122.809) (width 0.6) (layer F.Cu) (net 2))
 (segment (start 130.175 109.474) (end 133.053 109.474) (width 0.6) (layer F.Cu) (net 2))
 (segment (start 133.053 109.474) (end 133.223 109.304) (width 0.6) (layer F.Cu) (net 2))
 (segment (start 115.654 112.268) (end 115.654 115.189) (width 0.6) (layer F.Cu) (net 14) (status 20))
 (segment (start 115.654 115.189) (end 117.305 114.3) (width 0.6) (layer F.Cu) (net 14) (status 10))
 (segment (start 117.305 114.3) (end 122.555 114.3) (width 0.6) (layer F.Cu) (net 14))
 (segment (start 114.47 106.487) (end 114.239 106.487) (width 0.6) (layer F.Cu) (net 11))
 (segment (start 114.239 106.487) (end 111.379 109.347) (width 0.6) (layer F.Cu) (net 11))
 (segment (start 111.379 109.347) (end 110.744 109.347) (width 0.6) (layer F.Cu) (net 11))
 (segment (start 108.839 104.267) (end 107.061 104.267) (width 0.6) (layer F.Cu) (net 11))
 (segment (start 107.188 109.347) (end 108.839 109.347) (width 0.6) (layer F.Cu) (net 11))
 (segment (start 106.299 108.458) (end 107.188 109.347) (width 0.6) (layer F.Cu) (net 11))
 (segment (start 106.299 105.029) (end 106.299 108.458) (width 0.6) (layer F.Cu) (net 11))
 (segment (start 107.061 104.267) (end 106.299 105.029) (width 0.6) (layer F.Cu) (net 11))
 (segment (start 111.76 104.587) (end 111.76 104.394) (width 0.6) (layer F.Cu) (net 11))
 (segment (start 111.76 104.394) (end 112.268 103.886) (width 0.6) (layer F.Cu) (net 11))
 (segment (start 114.47 104.183) (end 114.47 104.587) (width 0.6) (layer F.Cu) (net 11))
 (segment (start 114.173 103.886) (end 114.47 104.183) (width 0.6) (layer F.Cu) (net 11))
 (segment (start 112.268 103.886) (end 114.173 103.886) (width 0.6) (layer F.Cu) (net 11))
 (segment (start 113.454 112.268) (end 111.76 112.268) (width 0.6) (layer F.Cu) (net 11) (status 10))
 (segment (start 108.839 114.681) (end 110.617 114.681) (width 0.6) (layer F.Cu) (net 11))
 (segment (start 110.744 109.347) (end 108.839 109.347) (width 0.6) (layer F.Cu) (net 11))
 (segment (start 111.76 112.268) (end 111.76 110.363) (width 0.6) (layer F.Cu) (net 11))
 (segment (start 111.76 110.363) (end 110.744 109.347) (width 0.6) (layer F.Cu) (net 11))
 (segment (start 111.76 113.538) (end 111.76 112.268) (width 0.6) (layer F.Cu) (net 11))
 (segment (start 110.617 114.681) (end 111.76 113.538) (width 0.6) (layer F.Cu) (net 11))
 (segment (start 108.839 104.267) (end 111.44 104.267) (width 0.6) (layer F.Cu) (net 11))
 (segment (start 111.44 104.267) (end 111.76 104.587) (width 0.6) (layer F.Cu) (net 11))
 (segment (start 128.778 89.027) (end 131.93 89.027) (width 0.6) (layer F.Cu) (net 7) (status 10))
 (segment (start 131.93 89.027) (end 133.139 90.236) (width 0.6) (layer F.Cu) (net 7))
 (segment (start 112.372 89.027) (end 113.581 90.236) (width 0.6) (layer F.Cu) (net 7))
 (segment (start 109.22 89.027) (end 112.372 89.027) (width 0.6) (layer F.Cu) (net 7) (status 10))
 (segment (start 133.139 92.136) (end 132.334 92.964) (width 0.6) (layer F.Cu) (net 6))
 (segment (start 132.334 92.964) (end 128.397 94.107) (width 0.6) (layer F.Cu) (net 6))
 (segment (start 112.776 92.964) (end 108.839 94.107) (width 0.6) (layer F.Cu) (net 6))
 (segment (start 113.581 92.136) (end 112.776 92.964) (width 0.6) (layer F.Cu) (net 6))
 (segment (start 139.573 117.475) (end 141.224 119.126) (width 0.6) (layer F.Cu) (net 4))
 (segment (start 130.175 117.475) (end 139.573 117.475) (width 0.6) (layer F.Cu) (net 4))
 (segment (start 130.175 104.14) (end 139.573 104.14) (width 0.6) (layer F.Cu) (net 4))
 (segment (start 139.573 104.14) (end 141.224 105.791) (width 0.6) (layer F.Cu) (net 4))
 (segment (start 137.455 122.217) (end 137.795 121.877) (width 0.6) (layer F.Cu) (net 5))
 (segment (start 135.636 122.217) (end 137.455 122.217) (width 0.6) (layer F.Cu) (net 5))
 (segment (start 141.013 121.877) (end 141.224 121.666) (width 0.6) (layer F.Cu) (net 5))
 (segment (start 137.795 121.877) (end 141.013 121.877) (width 0.6) (layer F.Cu) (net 5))
 (segment (start 137.795 108.542) (end 141.013 108.542) (width 0.6) (layer F.Cu) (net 5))
 (segment (start 141.013 108.542) (end 141.224 108.331) (width 0.6) (layer F.Cu) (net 5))
 (segment (start 135.636 108.882) (end 137.455 108.882) (width 0.6) (layer F.Cu) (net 5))
 (segment (start 137.455 108.882) (end 137.795 108.542) (width 0.6) (layer F.Cu) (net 5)))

